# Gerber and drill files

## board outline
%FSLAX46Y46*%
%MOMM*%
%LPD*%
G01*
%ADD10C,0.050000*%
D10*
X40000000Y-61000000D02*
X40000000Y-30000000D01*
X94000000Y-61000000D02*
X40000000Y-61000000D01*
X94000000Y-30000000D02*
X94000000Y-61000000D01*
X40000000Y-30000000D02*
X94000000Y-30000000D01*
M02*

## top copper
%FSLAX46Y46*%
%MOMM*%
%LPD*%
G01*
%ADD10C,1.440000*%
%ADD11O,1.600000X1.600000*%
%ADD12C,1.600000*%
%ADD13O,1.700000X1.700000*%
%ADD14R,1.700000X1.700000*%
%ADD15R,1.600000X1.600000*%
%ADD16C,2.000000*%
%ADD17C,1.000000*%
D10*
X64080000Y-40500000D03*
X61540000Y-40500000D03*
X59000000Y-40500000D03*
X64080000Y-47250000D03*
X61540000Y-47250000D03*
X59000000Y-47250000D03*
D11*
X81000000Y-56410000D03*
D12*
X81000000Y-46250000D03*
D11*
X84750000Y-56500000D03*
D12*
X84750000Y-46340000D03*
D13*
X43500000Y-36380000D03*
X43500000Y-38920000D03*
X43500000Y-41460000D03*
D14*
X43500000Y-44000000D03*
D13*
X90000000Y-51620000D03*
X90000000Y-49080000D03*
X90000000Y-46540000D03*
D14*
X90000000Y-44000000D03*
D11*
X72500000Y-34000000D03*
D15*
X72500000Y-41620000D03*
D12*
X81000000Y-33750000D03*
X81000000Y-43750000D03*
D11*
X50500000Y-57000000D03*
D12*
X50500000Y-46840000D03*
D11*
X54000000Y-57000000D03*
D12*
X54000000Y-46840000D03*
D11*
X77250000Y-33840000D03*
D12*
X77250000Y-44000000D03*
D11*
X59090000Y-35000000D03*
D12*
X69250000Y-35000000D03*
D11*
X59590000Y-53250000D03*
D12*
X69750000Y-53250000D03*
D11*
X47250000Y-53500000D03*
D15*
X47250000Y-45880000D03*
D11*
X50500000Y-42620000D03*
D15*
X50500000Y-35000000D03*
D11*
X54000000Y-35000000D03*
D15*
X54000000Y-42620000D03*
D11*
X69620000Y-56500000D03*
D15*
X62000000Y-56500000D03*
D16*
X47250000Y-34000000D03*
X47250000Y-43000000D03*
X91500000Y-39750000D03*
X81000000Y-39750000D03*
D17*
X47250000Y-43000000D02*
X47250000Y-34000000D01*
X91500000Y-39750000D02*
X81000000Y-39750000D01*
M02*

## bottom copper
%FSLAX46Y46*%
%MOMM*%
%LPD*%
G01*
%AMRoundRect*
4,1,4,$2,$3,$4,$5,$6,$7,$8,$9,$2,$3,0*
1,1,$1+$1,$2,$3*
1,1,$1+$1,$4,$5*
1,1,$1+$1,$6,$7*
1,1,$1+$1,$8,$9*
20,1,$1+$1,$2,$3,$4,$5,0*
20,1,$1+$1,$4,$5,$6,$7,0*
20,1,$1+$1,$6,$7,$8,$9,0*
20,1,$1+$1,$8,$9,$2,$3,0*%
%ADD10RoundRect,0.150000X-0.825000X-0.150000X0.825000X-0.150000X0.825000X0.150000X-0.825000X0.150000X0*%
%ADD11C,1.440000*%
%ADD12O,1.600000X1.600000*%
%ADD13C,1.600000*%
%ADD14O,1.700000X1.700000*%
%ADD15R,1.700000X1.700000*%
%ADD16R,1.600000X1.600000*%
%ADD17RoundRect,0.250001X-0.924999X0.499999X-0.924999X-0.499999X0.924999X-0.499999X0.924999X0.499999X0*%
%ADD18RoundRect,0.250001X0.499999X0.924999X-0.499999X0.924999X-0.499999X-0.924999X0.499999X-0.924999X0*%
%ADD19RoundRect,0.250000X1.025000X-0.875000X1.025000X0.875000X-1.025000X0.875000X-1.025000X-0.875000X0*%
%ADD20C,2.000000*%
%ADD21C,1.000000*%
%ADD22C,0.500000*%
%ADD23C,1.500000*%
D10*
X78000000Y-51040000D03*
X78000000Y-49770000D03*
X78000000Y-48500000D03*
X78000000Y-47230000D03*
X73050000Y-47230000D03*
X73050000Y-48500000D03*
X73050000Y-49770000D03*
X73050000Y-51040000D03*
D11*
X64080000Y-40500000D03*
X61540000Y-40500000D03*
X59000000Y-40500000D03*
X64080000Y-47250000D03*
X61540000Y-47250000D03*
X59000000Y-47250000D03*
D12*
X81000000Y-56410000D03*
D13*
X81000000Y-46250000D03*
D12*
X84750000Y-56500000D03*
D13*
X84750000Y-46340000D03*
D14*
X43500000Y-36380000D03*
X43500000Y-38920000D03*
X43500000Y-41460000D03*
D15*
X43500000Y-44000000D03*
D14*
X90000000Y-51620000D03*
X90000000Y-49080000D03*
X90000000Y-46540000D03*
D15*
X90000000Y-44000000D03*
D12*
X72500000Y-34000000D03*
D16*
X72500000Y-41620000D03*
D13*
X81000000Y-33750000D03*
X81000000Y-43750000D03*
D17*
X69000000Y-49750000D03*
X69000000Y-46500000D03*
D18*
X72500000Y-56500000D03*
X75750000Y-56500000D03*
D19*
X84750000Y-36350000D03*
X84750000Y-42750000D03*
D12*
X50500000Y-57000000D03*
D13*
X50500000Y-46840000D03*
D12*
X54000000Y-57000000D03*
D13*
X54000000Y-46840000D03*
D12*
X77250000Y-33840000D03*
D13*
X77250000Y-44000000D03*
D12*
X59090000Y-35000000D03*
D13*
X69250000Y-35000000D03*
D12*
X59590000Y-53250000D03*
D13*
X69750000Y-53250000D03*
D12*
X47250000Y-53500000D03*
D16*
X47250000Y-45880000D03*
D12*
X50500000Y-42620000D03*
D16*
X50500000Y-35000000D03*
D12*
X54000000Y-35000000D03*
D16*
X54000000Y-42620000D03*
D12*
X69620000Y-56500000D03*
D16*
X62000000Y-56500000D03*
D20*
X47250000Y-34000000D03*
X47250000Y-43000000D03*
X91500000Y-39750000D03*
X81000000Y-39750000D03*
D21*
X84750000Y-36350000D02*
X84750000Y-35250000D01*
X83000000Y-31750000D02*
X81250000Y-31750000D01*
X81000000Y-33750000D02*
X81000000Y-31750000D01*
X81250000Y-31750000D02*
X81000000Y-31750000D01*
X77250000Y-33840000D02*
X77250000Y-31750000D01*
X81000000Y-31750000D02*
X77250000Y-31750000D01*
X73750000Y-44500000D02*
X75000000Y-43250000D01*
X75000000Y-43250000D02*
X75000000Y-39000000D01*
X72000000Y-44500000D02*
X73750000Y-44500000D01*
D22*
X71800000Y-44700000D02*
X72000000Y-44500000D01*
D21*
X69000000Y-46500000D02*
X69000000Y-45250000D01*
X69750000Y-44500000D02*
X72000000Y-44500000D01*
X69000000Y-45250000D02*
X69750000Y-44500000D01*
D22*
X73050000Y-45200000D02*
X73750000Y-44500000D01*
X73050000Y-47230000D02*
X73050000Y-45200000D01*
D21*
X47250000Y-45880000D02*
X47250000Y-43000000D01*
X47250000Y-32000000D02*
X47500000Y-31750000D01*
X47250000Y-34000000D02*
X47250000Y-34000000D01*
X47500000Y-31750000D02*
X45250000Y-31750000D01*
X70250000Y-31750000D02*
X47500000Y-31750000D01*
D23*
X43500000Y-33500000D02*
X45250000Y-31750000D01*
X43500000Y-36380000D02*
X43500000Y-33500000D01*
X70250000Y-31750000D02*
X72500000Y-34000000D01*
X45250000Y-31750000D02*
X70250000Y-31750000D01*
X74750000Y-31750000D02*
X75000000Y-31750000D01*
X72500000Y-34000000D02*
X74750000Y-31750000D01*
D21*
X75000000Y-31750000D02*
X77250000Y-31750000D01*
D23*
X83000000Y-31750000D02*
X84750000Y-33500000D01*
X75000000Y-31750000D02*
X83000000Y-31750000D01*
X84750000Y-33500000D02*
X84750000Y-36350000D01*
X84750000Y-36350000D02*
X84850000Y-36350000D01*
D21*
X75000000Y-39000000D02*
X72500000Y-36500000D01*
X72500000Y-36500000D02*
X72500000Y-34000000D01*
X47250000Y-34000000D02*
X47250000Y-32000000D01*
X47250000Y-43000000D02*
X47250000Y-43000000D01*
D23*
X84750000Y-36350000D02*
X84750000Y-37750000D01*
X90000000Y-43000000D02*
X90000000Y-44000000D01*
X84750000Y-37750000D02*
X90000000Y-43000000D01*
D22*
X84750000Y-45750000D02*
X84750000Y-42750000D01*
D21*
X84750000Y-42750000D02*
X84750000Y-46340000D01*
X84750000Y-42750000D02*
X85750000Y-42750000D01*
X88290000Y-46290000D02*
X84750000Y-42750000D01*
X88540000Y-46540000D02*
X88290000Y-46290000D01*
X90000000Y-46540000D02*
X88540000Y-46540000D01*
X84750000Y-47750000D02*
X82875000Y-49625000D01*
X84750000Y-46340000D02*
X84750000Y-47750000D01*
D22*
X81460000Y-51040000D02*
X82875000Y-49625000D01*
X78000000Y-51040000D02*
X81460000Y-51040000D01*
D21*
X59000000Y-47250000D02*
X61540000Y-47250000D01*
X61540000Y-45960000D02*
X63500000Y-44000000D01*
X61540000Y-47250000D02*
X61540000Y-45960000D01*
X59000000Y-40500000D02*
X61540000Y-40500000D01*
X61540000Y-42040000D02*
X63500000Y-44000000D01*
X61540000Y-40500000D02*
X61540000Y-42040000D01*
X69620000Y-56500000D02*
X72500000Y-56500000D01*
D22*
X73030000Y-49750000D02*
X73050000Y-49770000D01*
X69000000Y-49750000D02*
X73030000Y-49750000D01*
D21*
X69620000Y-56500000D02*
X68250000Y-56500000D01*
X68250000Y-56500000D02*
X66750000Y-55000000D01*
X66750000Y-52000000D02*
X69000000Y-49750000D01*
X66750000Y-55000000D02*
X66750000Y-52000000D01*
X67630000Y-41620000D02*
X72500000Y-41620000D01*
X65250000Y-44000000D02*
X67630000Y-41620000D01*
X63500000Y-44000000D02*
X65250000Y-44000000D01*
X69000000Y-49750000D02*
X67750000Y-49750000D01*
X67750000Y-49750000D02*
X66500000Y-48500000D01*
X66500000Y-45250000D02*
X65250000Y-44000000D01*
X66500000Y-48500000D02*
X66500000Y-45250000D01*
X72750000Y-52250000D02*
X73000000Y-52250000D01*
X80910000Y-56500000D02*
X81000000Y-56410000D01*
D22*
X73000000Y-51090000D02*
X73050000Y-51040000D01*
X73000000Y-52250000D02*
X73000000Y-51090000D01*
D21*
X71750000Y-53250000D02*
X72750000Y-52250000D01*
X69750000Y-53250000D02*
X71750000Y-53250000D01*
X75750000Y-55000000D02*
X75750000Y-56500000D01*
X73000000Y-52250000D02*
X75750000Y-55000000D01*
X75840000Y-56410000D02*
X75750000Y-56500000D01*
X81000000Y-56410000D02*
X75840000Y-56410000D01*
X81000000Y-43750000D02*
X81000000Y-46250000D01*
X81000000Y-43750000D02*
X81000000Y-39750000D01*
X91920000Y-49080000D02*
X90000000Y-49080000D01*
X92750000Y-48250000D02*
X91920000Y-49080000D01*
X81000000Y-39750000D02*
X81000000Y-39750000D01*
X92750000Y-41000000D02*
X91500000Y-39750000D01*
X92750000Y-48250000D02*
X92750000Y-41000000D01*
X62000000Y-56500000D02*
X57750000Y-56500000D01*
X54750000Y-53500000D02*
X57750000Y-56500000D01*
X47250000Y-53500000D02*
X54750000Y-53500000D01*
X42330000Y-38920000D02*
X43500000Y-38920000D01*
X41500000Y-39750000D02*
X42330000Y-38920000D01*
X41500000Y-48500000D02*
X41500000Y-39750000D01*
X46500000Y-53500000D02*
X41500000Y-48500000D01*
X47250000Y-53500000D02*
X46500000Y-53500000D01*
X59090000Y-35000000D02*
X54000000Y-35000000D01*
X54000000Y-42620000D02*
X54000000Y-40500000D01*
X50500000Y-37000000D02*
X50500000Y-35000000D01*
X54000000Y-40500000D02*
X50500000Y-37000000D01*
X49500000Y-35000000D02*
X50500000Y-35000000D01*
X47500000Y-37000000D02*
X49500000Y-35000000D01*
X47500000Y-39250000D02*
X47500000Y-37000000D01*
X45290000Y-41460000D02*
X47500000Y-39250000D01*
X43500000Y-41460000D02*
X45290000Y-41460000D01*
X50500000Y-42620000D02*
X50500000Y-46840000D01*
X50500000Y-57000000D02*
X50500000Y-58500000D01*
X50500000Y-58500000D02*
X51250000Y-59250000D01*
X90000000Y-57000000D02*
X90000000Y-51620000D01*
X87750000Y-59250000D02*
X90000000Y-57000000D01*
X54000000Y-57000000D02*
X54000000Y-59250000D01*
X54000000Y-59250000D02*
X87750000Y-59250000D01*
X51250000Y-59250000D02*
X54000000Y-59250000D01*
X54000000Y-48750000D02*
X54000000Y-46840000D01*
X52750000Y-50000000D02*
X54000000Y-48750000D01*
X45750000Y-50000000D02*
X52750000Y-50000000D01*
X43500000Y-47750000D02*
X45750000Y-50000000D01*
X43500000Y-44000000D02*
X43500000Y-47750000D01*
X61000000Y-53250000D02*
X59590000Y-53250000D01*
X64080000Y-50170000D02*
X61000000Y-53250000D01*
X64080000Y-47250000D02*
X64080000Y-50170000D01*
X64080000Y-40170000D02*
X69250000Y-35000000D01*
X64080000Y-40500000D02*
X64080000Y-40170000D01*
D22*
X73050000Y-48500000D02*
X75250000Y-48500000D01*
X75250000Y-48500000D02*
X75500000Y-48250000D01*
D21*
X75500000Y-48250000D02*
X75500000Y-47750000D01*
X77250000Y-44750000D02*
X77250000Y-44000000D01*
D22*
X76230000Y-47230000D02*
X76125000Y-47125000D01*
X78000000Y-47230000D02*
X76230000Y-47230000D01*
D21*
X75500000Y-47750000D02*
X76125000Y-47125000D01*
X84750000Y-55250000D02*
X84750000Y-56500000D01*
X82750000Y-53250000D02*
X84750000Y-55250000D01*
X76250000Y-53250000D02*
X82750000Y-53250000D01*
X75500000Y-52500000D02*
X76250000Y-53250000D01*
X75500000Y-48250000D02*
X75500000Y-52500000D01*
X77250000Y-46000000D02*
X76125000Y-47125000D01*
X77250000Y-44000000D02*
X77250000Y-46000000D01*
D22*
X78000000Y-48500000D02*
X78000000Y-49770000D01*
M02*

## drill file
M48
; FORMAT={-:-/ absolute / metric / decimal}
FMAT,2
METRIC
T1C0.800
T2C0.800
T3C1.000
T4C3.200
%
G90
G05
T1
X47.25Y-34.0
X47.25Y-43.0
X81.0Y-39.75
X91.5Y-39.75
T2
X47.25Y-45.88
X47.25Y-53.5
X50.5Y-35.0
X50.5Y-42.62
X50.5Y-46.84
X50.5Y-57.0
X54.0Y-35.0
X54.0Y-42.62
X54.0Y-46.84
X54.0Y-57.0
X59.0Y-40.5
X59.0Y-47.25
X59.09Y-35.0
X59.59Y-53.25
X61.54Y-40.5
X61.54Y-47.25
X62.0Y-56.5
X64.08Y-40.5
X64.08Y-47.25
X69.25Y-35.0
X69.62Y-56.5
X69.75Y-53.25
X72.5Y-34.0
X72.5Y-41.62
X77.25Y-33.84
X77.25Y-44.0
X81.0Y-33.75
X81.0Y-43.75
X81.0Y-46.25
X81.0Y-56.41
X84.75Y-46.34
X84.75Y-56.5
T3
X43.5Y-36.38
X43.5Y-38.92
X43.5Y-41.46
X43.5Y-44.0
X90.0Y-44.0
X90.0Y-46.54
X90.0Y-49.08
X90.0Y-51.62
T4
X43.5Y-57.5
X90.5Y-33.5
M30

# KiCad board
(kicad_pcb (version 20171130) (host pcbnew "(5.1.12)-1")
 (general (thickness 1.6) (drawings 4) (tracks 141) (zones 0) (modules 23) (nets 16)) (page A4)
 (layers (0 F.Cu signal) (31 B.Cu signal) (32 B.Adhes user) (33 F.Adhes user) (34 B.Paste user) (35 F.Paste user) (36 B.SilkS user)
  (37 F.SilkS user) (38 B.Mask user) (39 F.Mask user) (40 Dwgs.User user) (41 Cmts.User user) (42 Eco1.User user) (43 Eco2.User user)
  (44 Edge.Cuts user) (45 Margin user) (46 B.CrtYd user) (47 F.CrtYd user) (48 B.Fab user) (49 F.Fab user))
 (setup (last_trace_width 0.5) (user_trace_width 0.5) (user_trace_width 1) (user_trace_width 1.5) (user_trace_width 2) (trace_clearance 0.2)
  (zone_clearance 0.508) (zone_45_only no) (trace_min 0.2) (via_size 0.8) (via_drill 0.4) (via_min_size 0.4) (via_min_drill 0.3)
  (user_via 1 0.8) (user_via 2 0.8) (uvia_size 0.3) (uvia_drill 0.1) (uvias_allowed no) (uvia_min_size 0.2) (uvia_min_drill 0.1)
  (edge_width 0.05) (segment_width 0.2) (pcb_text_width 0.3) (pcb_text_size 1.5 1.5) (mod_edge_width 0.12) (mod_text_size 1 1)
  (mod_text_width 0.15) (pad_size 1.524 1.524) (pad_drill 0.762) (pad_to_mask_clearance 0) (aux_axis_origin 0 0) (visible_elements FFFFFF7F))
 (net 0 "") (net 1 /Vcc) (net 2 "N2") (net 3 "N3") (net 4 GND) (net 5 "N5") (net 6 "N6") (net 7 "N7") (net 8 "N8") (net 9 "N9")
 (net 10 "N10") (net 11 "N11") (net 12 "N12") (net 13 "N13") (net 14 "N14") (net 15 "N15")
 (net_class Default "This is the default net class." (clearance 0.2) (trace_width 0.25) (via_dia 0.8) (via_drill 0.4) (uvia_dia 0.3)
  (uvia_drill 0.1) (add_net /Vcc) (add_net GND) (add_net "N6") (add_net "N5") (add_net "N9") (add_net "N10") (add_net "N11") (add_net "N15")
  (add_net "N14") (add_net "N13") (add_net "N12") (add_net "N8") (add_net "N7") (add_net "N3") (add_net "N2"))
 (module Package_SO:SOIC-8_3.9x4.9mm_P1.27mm (layer B.Cu) (at 75.525 49.135)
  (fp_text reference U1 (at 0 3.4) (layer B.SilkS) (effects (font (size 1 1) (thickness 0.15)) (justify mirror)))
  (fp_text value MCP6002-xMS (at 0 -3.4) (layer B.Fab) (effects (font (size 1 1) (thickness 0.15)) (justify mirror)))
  (pad 8 smd roundrect (at 2.475 1.905) (size 1.95 0.6) (layers B.Cu B.Paste B.Mask) (roundrect_rratio 0.25) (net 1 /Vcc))
  (pad 7 smd roundrect (at 2.475 0.635) (size 1.95 0.6) (layers B.Cu B.Paste B.Mask) (roundrect_rratio 0.25) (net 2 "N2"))
  (pad 6 smd roundrect (at 2.475 -0.635) (size 1.95 0.6) (layers B.Cu B.Paste B.Mask) (roundrect_rratio 0.25) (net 2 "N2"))
  (pad 5 smd roundrect (at 2.475 -1.905) (size 1.95 0.6) (layers B.Cu B.Paste B.Mask) (roundrect_rratio 0.25) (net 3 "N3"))
  (pad 4 smd roundrect (at -2.475 -1.905) (size 1.95 0.6) (layers B.Cu B.Paste B.Mask) (roundrect_rratio 0.25) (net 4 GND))
  (pad 3 smd roundrect (at -2.475 -0.635) (size 1.95 0.6) (layers B.Cu B.Paste B.Mask) (roundrect_rratio 0.25) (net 3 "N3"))
  (pad 2 smd roundrect (at -2.475 0.635) (size 1.95 0.6) (layers B.Cu B.Paste B.Mask) (roundrect_rratio 0.25) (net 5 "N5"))
  (pad 1 smd roundrect (at -2.475 1.905) (size 1.95 0.6) (layers B.Cu B.Paste B.Mask) (roundrect_rratio 0.25) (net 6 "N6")))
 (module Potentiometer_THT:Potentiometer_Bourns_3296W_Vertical (layer F.Cu) (at 59 40.5 180)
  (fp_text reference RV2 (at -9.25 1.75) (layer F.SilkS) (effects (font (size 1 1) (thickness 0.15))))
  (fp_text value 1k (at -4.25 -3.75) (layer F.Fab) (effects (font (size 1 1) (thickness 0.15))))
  (pad 3 thru_hole circle (at -5.08 0 180) (size 1.44 1.44) (drill 0.8) (layers *.Cu *.Mask) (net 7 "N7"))
  (pad 2 thru_hole circle (at -2.54 0 180) (size 1.44 1.44) (drill 0.8) (layers *.Cu *.Mask) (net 5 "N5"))
  (pad 1 thru_hole circle (at 0 0 180) (size 1.44 1.44) (drill 0.8) (layers *.Cu *.Mask) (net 5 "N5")))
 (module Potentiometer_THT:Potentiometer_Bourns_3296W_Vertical (layer F.Cu) (at 59 47.25 180)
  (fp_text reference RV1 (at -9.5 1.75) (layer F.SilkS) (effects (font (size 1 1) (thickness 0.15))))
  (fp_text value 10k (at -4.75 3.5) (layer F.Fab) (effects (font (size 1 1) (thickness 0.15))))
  (pad 3 thru_hole circle (at -5.08 0 180) (size 1.44 1.44) (drill 0.8) (layers *.Cu *.Mask) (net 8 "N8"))
  (pad 2 thru_hole circle (at -2.54 0 180) (size 1.44 1.44) (drill 0.8) (layers *.Cu *.Mask) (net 5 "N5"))
  (pad 1 thru_hole circle (at 0 0 180) (size 1.44 1.44) (drill 0.8) (layers *.Cu *.Mask) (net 5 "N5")))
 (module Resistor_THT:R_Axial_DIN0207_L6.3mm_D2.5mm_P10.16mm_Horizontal (layer F.Cu) (at 81 46.25 270)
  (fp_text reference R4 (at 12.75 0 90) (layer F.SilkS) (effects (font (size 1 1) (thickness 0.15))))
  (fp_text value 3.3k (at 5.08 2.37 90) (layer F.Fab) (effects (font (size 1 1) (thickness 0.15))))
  (pad 2 thru_hole oval (at 10.16 0 270) (size 1.6 1.6) (drill 0.8) (layers *.Cu *.Mask) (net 6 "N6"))
  (pad 1 thru_hole circle (at 0 0 270) (size 1.6 1.6) (drill 0.8) (layers *.Cu *.Mask) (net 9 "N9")))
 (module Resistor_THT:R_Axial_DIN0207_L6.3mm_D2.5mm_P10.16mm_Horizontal (layer F.Cu) (at 84.75 46.34 270)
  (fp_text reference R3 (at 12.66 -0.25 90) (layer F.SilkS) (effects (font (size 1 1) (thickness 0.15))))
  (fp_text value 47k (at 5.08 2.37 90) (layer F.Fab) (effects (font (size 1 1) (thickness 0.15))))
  (pad 2 thru_hole oval (at 10.16 0 270) (size 1.6 1.6) (drill 0.8) (layers *.Cu *.Mask) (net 3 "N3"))
  (pad 1 thru_hole circle (at 0 0 270) (size 1.6 1.6) (drill 0.8) (layers *.Cu *.Mask) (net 1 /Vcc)))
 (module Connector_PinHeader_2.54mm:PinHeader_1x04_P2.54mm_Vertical (layer F.Cu) (at 43.5 44 180)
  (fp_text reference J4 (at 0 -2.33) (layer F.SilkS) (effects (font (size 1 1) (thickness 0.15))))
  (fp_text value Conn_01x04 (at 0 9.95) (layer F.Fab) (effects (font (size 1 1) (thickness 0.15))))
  (pad 4 thru_hole oval (at 0 7.62 180) (size 1.7 1.7) (drill 1) (layers *.Cu *.Mask) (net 4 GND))
  (pad 3 thru_hole oval (at 0 5.08 180) (size 1.7 1.7) (drill 1) (layers *.Cu *.Mask) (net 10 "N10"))
  (pad 2 thru_hole oval (at 0 2.54 180) (size 1.7 1.7) (drill 1) (layers *.Cu *.Mask) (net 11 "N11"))
  (pad 1 thru_hole rect (at 0 0 180) (size 1.7 1.7) (drill 1) (layers *.Cu *.Mask) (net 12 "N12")))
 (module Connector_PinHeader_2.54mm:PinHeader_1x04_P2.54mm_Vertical (layer F.Cu) (at 90 44)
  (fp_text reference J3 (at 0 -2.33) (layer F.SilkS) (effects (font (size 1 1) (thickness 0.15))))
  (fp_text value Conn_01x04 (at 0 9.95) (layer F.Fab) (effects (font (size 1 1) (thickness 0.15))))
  (pad 4 thru_hole oval (at 0 7.62) (size 1.7 1.7) (drill 1) (layers *.Cu *.Mask) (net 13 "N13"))
  (pad 3 thru_hole oval (at 0 5.08) (size 1.7 1.7) (drill 1) (layers *.Cu *.Mask) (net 9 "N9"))
  (pad 2 thru_hole oval (at 0 2.54) (size 1.7 1.7) (drill 1) (layers *.Cu *.Mask) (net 1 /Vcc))
  (pad 1 thru_hole rect (at 0 0) (size 1.7 1.7) (drill 1) (layers *.Cu *.Mask) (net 4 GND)))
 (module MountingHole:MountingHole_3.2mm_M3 (layer F.Cu) (at 90.5 33.5)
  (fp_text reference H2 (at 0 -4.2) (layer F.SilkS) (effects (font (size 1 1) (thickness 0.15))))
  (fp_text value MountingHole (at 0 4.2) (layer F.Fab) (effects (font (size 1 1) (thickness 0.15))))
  (pad 1 np_thru_hole circle (at 0 0) (size 3.2 3.2) (drill 3.2) (layers *.Cu *.Mask)))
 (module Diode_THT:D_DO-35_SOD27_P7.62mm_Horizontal (layer F.Cu) (at 72.5 41.62 90)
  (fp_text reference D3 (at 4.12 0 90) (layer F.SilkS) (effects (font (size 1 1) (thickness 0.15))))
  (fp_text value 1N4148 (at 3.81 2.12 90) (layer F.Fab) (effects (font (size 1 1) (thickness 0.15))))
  (pad 2 thru_hole oval (at 7.62 0 90) (size 1.6 1.6) (drill 0.8) (layers *.Cu *.Mask) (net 4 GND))
  (pad 1 thru_hole rect (at 0 0 90) (size 1.6 1.6) (drill 0.8) (layers *.Cu *.Mask) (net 5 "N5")))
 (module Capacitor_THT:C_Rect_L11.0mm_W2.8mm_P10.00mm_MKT (layer F.Cu) (at 81 43.75 90)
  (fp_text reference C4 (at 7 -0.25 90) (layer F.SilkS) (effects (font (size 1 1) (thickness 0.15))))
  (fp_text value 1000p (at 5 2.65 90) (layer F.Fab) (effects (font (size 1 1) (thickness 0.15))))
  (pad 2 thru_hole circle (at 10 0 90) (size 1.6 1.6) (drill 0.8) (layers *.Cu *.Mask) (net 4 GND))
  (pad 1 thru_hole circle (at 0 0 90) (size 1.6 1.6) (drill 0.8) (layers *.Cu *.Mask) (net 9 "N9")))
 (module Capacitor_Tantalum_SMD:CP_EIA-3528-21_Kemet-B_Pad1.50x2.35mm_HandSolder (layer B.Cu) (at 69 48.125 270)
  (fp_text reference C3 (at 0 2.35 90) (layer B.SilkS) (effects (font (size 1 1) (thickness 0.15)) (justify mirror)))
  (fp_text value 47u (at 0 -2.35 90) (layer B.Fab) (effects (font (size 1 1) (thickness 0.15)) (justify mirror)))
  (pad 2 smd roundrect (at 1.625 0 270) (size 1.5 2.35) (layers B.Cu B.Paste B.Mask) (roundrect_rratio 0.166667) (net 5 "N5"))
  (pad 1 smd roundrect (at -1.625 0 270) (size 1.5 2.35) (layers B.Cu B.Paste B.Mask) (roundrect_rratio 0.166667) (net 4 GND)))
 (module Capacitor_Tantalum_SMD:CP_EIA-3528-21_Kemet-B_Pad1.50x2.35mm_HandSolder (layer B.Cu) (at 74.125 56.5 180)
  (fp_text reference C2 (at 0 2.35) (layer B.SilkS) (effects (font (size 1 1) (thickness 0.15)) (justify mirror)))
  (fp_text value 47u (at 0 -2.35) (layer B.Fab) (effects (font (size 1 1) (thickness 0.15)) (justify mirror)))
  (pad 2 smd roundrect (at 1.625 0 180) (size 1.5 2.35) (layers B.Cu B.Paste B.Mask) (roundrect_rratio 0.166667) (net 5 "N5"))
  (pad 1 smd roundrect (at -1.625 0 180) (size 1.5 2.35) (layers B.Cu B.Paste B.Mask) (roundrect_rratio 0.166667) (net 6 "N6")))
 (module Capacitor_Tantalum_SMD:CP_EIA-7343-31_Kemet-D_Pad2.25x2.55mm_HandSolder (layer B.Cu) (at 84.75 39.55 90)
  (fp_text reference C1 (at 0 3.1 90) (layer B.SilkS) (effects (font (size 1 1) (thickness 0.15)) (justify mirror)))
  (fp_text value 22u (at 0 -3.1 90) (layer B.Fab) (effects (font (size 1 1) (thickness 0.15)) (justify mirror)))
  (pad 2 smd roundrect (at 3.2 0 90) (size 2.25 2.55) (layers B.Cu B.Paste B.Mask) (roundrect_rratio 0.111111) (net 4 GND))
  (pad 1 smd roundrect (at -3.2 0 90) (size 2.25 2.55) (layers B.Cu B.Paste B.Mask) (roundrect_rratio 0.111111) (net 1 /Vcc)))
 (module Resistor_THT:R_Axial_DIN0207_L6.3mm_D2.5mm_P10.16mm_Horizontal (layer F.Cu) (at 50.5 46.84 270)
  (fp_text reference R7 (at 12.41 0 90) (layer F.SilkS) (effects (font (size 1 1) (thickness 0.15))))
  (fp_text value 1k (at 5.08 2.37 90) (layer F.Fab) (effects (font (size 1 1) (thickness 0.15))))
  (pad 2 thru_hole oval (at 10.16 0 270) (size 1.6 1.6) (drill 0.8) (layers *.Cu *.Mask) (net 13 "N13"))
  (pad 1 thru_hole circle (at 0 0 270) (size 1.6 1.6) (drill 0.8) (layers *.Cu *.Mask) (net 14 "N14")))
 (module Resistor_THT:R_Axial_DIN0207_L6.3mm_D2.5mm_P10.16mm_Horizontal (layer F.Cu) (at 54 46.84 270)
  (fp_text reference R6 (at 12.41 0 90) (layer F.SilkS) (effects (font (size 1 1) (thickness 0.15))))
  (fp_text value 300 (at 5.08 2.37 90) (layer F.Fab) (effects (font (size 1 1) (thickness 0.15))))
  (pad 2 thru_hole oval (at 10.16 0 270) (size 1.6 1.6) (drill 0.8) (layers *.Cu *.Mask) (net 13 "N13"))
  (pad 1 thru_hole circle (at 0 0 270) (size 1.6 1.6) (drill 0.8) (layers *.Cu *.Mask) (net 12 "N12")))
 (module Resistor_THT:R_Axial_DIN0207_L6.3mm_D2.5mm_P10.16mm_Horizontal (layer F.Cu) (at 77.25 44 90)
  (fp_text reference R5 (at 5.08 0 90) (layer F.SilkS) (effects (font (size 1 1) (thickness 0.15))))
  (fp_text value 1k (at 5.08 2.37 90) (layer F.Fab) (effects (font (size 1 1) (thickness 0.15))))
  (pad 2 thru_hole oval (at 10.16 0 90) (size 1.6 1.6) (drill 0.8) (layers *.Cu *.Mask) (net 4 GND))
  (pad 1 thru_hole circle (at 0 0 90) (size 1.6 1.6) (drill 0.8) (layers *.Cu *.Mask) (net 3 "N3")))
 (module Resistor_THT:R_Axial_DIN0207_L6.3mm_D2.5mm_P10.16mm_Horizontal (layer F.Cu) (at 69.25 35 180)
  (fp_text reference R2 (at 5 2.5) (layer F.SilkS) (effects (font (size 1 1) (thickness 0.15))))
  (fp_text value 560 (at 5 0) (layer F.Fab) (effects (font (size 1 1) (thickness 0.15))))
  (pad 2 thru_hole oval (at 10.16 0 180) (size 1.6 1.6) (drill 0.8) (layers *.Cu *.Mask) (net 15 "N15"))
  (pad 1 thru_hole circle (at 0 0 180) (size 1.6 1.6) (drill 0.8) (layers *.Cu *.Mask) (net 7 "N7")))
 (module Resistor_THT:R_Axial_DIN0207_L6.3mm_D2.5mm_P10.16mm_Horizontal (layer F.Cu) (at 69.75 53.25 180)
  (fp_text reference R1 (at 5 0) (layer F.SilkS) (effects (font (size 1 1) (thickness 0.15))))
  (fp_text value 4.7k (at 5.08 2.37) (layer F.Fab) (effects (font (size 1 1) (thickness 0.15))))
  (pad 2 thru_hole oval (at 10.16 0 180) (size 1.6 1.6) (drill 0.8) (layers *.Cu *.Mask) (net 8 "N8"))
  (pad 1 thru_hole circle (at 0 0 180) (size 1.6 1.6) (drill 0.8) (layers *.Cu *.Mask) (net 6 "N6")))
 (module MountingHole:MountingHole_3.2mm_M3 (layer F.Cu) (at 43.5 57.5)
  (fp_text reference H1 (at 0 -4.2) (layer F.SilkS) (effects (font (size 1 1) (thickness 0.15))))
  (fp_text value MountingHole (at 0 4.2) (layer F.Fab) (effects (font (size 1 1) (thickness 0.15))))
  (pad 1 np_thru_hole circle (at 0 0) (size 3.2 3.2) (drill 3.2) (layers *.Cu *.Mask)))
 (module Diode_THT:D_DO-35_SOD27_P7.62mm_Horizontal (layer F.Cu) (at 47.25 45.88 270)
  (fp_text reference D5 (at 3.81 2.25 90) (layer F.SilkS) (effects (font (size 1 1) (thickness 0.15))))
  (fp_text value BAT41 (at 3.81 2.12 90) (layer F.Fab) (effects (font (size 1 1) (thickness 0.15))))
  (pad 2 thru_hole oval (at 7.62 0 270) (size 1.6 1.6) (drill 0.8) (layers *.Cu *.Mask) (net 10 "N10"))
  (pad 1 thru_hole rect (at 0 0 270) (size 1.6 1.6) (drill 0.8) (layers *.Cu *.Mask) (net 4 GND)))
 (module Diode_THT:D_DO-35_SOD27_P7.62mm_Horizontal (layer F.Cu) (at 50.5 35 270)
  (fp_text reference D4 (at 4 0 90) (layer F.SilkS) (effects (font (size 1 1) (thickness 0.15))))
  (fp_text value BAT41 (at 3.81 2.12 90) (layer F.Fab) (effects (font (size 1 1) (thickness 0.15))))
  (pad 2 thru_hole oval (at 7.62 0 270) (size 1.6 1.6) (drill 0.8) (layers *.Cu *.Mask) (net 14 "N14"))
  (pad 1 thru_hole rect (at 0 0 270) (size 1.6 1.6) (drill 0.8) (layers *.Cu *.Mask) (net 11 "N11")))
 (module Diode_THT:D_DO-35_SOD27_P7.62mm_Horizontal (layer F.Cu) (at 54 42.62 90)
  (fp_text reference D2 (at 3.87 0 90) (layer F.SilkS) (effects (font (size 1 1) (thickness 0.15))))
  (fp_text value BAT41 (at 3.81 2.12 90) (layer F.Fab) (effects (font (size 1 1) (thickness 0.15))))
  (pad 2 thru_hole oval (at 7.62 0 90) (size 1.6 1.6) (drill 0.8) (layers *.Cu *.Mask) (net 15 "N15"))
  (pad 1 thru_hole rect (at 0 0 90) (size 1.6 1.6) (drill 0.8) (layers *.Cu *.Mask) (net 11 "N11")))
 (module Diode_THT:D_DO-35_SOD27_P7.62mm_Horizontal (layer F.Cu) (at 62 56.5)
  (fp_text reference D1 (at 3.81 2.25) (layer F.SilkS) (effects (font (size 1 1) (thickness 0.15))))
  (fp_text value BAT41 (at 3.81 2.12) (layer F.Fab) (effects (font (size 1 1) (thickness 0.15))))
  (pad 2 thru_hole oval (at 7.62 0) (size 1.6 1.6) (drill 0.8) (layers *.Cu *.Mask) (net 5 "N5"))
  (pad 1 thru_hole rect (at 0 0) (size 1.6 1.6) (drill 0.8) (layers *.Cu *.Mask) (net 10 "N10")))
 (gr_line (start 40 61) (end 40 30) (layer Edge.Cuts) (width 0.05))
 (gr_line (start 94 61) (end 40 61) (layer Edge.Cuts) (width 0.05))
 (gr_line (start 94 30) (end 94 61) (layer Edge.Cuts) (width 0.05))
 (gr_line (start 40 30) (end 94 30) (layer Edge.Cuts) (width 0.05))
 (segment (start 84.75 36.35) (end 84.75 35.25) (width 1) (layer B.Cu) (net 4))
 (segment (start 83 31.75) (end 81.25 31.75) (width 1) (layer B.Cu) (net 4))
 (segment (start 81 33.75) (end 81 31.75) (width 1) (layer B.Cu) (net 4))
 (segment (start 81.25 31.75) (end 81 31.75) (width 1) (layer B.Cu) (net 4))
 (segment (start 77.25 33.84) (end 77.25 31.75) (width 1) (layer B.Cu) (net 4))
 (segment (start 81 31.75) (end 77.25 31.75) (width 1) (layer B.Cu) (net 4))
 (segment (start 73.75 44.5) (end 75 43.25) (width 1) (layer B.Cu) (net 4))
 (segment (start 75 43.25) (end 75 39) (width 1) (layer B.Cu) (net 4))
 (segment (start 72 44.5) (end 73.75 44.5) (width 1) (layer B.Cu) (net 4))
 (segment (start 71.8 44.7) (end 72 44.5) (width 0.5) (layer B.Cu) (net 4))
 (segment (start 69 46.5) (end 69 45.25) (width 1) (layer B.Cu) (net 4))
 (segment (start 69.75 44.5) (end 72 44.5) (width 1) (layer B.Cu) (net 4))
 (segment (start 69 45.25) (end 69.75 44.5) (width 1) (layer B.Cu) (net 4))
 (segment (start 73.05 45.2) (end 73.75 44.5) (width 0.5) (layer B.Cu) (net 4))
 (segment (start 73.05 47.23) (end 73.05 45.2) (width 0.5) (layer B.Cu) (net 4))
 (segment (start 47.25 45.88) (end 47.25 43) (width 1) (layer B.Cu) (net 4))
 (segment (start 47.25 43) (end 47.25 34) (width 1) (layer F.Cu) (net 4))
 (segment (start 47.25 32) (end 47.5 31.75) (width 1) (layer B.Cu) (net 4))
 (segment (start 47.25 34) (end 47.25 34) (width 1) (layer B.Cu) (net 4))
 (segment (start 47.5 31.75) (end 45.25 31.75) (width 1) (layer B.Cu) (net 4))
 (segment (start 70.25 31.75) (end 47.5 31.75) (width 1) (layer B.Cu) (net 4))
 (segment (start 43.5 33.5) (end 45.25 31.75) (width 1.5) (layer B.Cu) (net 4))
 (segment (start 43.5 36.38) (end 43.5 33.5) (width 1.5) (layer B.Cu) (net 4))
 (segment (start 70.25 31.75) (end 72.5 34) (width 1.5) (layer B.Cu) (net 4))
 (segment (start 45.25 31.75) (end 70.25 31.75) (width 1.5) (layer B.Cu) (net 4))
 (segment (start 74.75 31.75) (end 75 31.75) (width 1.5) (layer B.Cu) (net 4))
 (segment (start 72.5 34) (end 74.75 31.75) (width 1.5) (layer B.Cu) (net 4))
 (segment (start 75 31.75) (end 77.25 31.75) (width 1) (layer B.Cu) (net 4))
 (segment (start 83 31.75) (end 84.75 33.5) (width 1.5) (layer B.Cu) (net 4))
 (segment (start 75 31.75) (end 83 31.75) (width 1.5) (layer B.Cu) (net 4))
 (segment (start 84.75 33.5) (end 84.75 36.35) (width 1.5) (layer B.Cu) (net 4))
 (segment (start 84.75 36.35) (end 84.85 36.35) (width 1.5) (layer B.Cu) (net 4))
 (segment (start 75 39) (end 72.5 36.5) (width 1) (layer B.Cu) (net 4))
 (segment (start 72.5 36.5) (end 72.5 34) (width 1) (layer B.Cu) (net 4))
 (segment (start 47.25 34) (end 47.25 32) (width 1) (layer B.Cu) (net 4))
 (via (at 47.25 34) (size 2) (drill 0.8) (layers F.Cu B.Cu) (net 4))
 (segment (start 47.25 43) (end 47.25 43) (width 1) (layer B.Cu) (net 4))
 (via (at 47.25 43) (size 2) (drill 0.8) (layers F.Cu B.Cu) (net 4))
 (segment (start 84.75 36.35) (end 84.75 37.75) (width 1.5) (layer B.Cu) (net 4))
 (segment (start 90 43) (end 90 44) (width 1.5) (layer B.Cu) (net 4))
 (segment (start 84.75 37.75) (end 90 43) (width 1.5) (layer B.Cu) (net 4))
 (segment (start 84.75 45.75) (end 84.75 42.75) (width 0.5) (layer B.Cu) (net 1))
 (segment (start 84.75 42.75) (end 84.75 46.34) (width 1) (layer B.Cu) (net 1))
 (segment (start 84.75 42.75) (end 85.75 42.75) (width 1) (layer B.Cu) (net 1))
 (segment (start 88.29 46.29) (end 84.75 42.75) (width 1) (layer B.Cu) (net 1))
 (segment (start 88.54 46.54) (end 88.29 46.29) (width 1) (layer B.Cu) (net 1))
 (segment (start 90 46.54) (end 88.54 46.54) (width 1) (layer B.Cu) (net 1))
 (segment (start 84.75 47.75) (end 82.875 49.625) (width 1) (layer B.Cu) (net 1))
 (segment (start 84.75 46.34) (end 84.75 47.75) (width 1) (layer B.Cu) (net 1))
 (segment (start 81.46 51.04) (end 82.875 49.625) (width 0.5) (layer B.Cu) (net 1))
 (segment (start 78 51.04) (end 81.46 51.04) (width 0.5) (layer B.Cu) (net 1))
 (segment (start 59 47.25) (end 61.54 47.25) (width 1) (layer B.Cu) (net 5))
 (segment (start 61.54 45.96) (end 63.5 44) (width 1) (layer B.Cu) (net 5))
 (segment (start 61.54 47.25) (end 61.54 45.96) (width 1) (layer B.Cu) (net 5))
 (segment (start 59 40.5) (end 61.54 40.5) (width 1) (layer B.Cu) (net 5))
 (segment (start 61.54 42.04) (end 63.5 44) (width 1) (layer B.Cu) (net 5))
 (segment (start 61.54 40.5) (end 61.54 42.04) (width 1) (layer B.Cu) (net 5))
 (segment (start 69.62 56.5) (end 72.5 56.5) (width 1) (layer B.Cu) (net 5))
 (segment (start 73.03 49.75) (end 73.05 49.77) (width 0.5) (layer B.Cu) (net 5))
 (segment (start 69 49.75) (end 73.03 49.75) (width 0.5) (layer B.Cu) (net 5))
 (segment (start 69.62 56.5) (end 68.25 56.5) (width 1) (layer B.Cu) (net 5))
 (segment (start 68.25 56.5) (end 66.75 55) (width 1) (layer B.Cu) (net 5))
 (segment (start 66.75 52) (end 69 49.75) (width 1) (layer B.Cu) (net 5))
 (segment (start 66.75 55) (end 66.75 52) (width 1) (layer B.Cu) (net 5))
 (segment (start 67.63 41.62) (end 72.5 41.62) (width 1) (layer B.Cu) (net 5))
 (segment (start 65.25 44) (end 67.63 41.62) (width 1) (layer B.Cu) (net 5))
 (segment (start 63.5 44) (end 65.25 44) (width 1) (layer B.Cu) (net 5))
 (segment (start 69 49.75) (end 67.75 49.75) (width 1) (layer B.Cu) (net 5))
 (segment (start 67.75 49.75) (end 66.5 48.5) (width 1) (layer B.Cu) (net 5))
 (segment (start 66.5 45.25) (end 65.25 44) (width 1) (layer B.Cu) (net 5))
 (segment (start 66.5 48.5) (end 66.5 45.25) (width 1) (layer B.Cu) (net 5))
 (segment (start 72.75 52.25) (end 73 52.25) (width 1) (layer B.Cu) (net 6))
 (segment (start 80.91 56.5) (end 81 56.41) (width 1) (layer B.Cu) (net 6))
 (segment (start 73 51.09) (end 73.05 51.04) (width 0.5) (layer B.Cu) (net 6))
 (segment (start 73 52.25) (end 73 51.09) (width 0.5) (layer B.Cu) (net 6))
 (segment (start 71.75 53.25) (end 72.75 52.25) (width 1) (layer B.Cu) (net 6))
 (segment (start 69.75 53.25) (end 71.75 53.25) (width 1) (layer B.Cu) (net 6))
 (segment (start 75.75 55) (end 75.75 56.5) (width 1) (layer B.Cu) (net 6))
 (segment (start 73 52.25) (end 75.75 55) (width 1) (layer B.Cu) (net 6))
 (segment (start 75.84 56.41) (end 75.75 56.5) (width 1) (layer B.Cu) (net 6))
 (segment (start 81 56.41) (end 75.84 56.41) (width 1) (layer B.Cu) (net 6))
 (segment (start 81 43.75) (end 81 46.25) (width 1) (layer B.Cu) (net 9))
 (segment (start 81 43.75) (end 81 39.75) (width 1) (layer B.Cu) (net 9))
 (segment (start 91.92 49.08) (end 90 49.08) (width 1) (layer B.Cu) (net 9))
 (segment (start 92.75 48.25) (end 91.92 49.08) (width 1) (layer B.Cu) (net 9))
 (via (at 91.5 39.75) (size 2) (drill 0.8) (layers F.Cu B.Cu) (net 9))
 (segment (start 81 39.75) (end 81 39.75) (width 1) (layer B.Cu) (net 9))
 (via (at 81 39.75) (size 2) (drill 0.8) (layers F.Cu B.Cu) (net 9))
 (segment (start 92.75 41) (end 91.5 39.75) (width 1) (layer B.Cu) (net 9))
 (segment (start 92.75 48.25) (end 92.75 41) (width 1) (layer B.Cu) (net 9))
 (segment (start 91.5 39.75) (end 81 39.75) (width 1) (layer F.Cu) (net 9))
 (segment (start 62 56.5) (end 57.75 56.5) (width 1) (layer B.Cu) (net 10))
 (segment (start 54.75 53.5) (end 57.75 56.5) (width 1) (layer B.Cu) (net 10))
 (segment (start 47.25 53.5) (end 54.75 53.5) (width 1) (layer B.Cu) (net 10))
 (segment (start 42.33 38.92) (end 43.5 38.92) (width 1) (layer B.Cu) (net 10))
 (segment (start 41.5 39.75) (end 42.33 38.92) (width 1) (layer B.Cu) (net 10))
 (segment (start 41.5 48.5) (end 41.5 39.75) (width 1) (layer B.Cu) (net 10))
 (segment (start 46.5 53.5) (end 41.5 48.5) (width 1) (layer B.Cu) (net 10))
 (segment (start 47.25 53.5) (end 46.5 53.5) (width 1) (layer B.Cu) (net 10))
 (segment (start 59.09 35) (end 54 35) (width 1) (layer B.Cu) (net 15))
 (segment (start 54 42.62) (end 54 40.5) (width 1) (layer B.Cu) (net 11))
 (segment (start 50.5 37) (end 50.5 35) (width 1) (layer B.Cu) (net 11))
 (segment (start 54 40.5) (end 50.5 37) (width 1) (layer B.Cu) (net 11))
 (segment (start 49.5 35) (end 50.5 35) (width 1) (layer B.Cu) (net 11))
 (segment (start 47.5 37) (end 49.5 35) (width 1) (layer B.Cu) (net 11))
 (segment (start 47.5 39.25) (end 47.5 37) (width 1) (layer B.Cu) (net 11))
 (segment (start 45.29 41.46) (end 47.5 39.25) (width 1) (layer B.Cu) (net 11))
 (segment (start 43.5 41.46) (end 45.29 41.46) (width 1) (layer B.Cu) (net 11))
 (segment (start 50.5 42.62) (end 50.5 46.84) (width 1) (layer B.Cu) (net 14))
 (segment (start 50.5 57) (end 50.5 58.5) (width 1) (layer B.Cu) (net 13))
 (segment (start 50.5 58.5) (end 51.25 59.25) (width 1) (layer B.Cu) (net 13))
 (segment (start 90 57) (end 90 51.62) (width 1) (layer B.Cu) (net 13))
 (segment (start 87.75 59.25) (end 90 57) (width 1) (layer B.Cu) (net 13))
 (segment (start 54 57) (end 54 59.25) (width 1) (layer B.Cu) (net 13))
 (segment (start 54 59.25) (end 87.75 59.25) (width 1) (layer B.Cu) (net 13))
 (segment (start 51.25 59.25) (end 54 59.25) (width 1) (layer B.Cu) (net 13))
 (segment (start 54 48.75) (end 54 46.84) (width 1) (layer B.Cu) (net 12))
 (segment (start 52.75 50) (end 54 48.75) (width 1) (layer B.Cu) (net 12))
 (segment (start 45.75 50) (end 52.75 50) (width 1) (layer B.Cu) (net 12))
 (segment (start 43.5 47.75) (end 45.75 50) (width 1) (layer B.Cu) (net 12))
 (segment (start 43.5 44) (end 43.5 47.75) (width 1) (layer B.Cu) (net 12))
 (segment (start 61 53.25) (end 59.59 53.25) (width 1) (layer B.Cu) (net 8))
 (segment (start 64.08 50.17) (end 61 53.25) (width 1) (layer B.Cu) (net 8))
 (segment (start 64.08 47.25) (end 64.08 50.17) (width 1) (layer B.Cu) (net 8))
 (segment (start 64.08 40.17) (end 69.25 35) (width 1) (layer B.Cu) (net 7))
 (segment (start 64.08 40.5) (end 64.08 40.17) (width 1) (layer B.Cu) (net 7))
 (segment (start 73.05 48.5) (end 75.25 48.5) (width 0.5) (layer B.Cu) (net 3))
 (segment (start 75.25 48.5) (end 75.5 48.25) (width 0.5) (layer B.Cu) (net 3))
 (segment (start 75.5 48.25) (end 75.5 47.75) (width 1) (layer B.Cu) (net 3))
 (segment (start 77.25 44.75) (end 77.25 44) (width 1) (layer B.Cu) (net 3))
 (segment (start 76.23 47.23) (end 76.125 47.125) (width 0.5) (layer B.Cu) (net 3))
 (segment (start 78 47.23) (end 76.23 47.23) (width 0.5) (layer B.Cu) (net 3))
 (segment (start 75.5 47.75) (end 76.125 47.125) (width 1) (layer B.Cu) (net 3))
 (segment (start 84.75 55.25) (end 84.75 56.5) (width 1) (layer B.Cu) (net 3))
 (segment (start 82.75 53.25) (end 84.75 55.25) (width 1) (layer B.Cu) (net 3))
 (segment (start 76.25 53.25) (end 82.75 53.25) (width 1) (layer B.Cu) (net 3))
 (segment (start 75.5 52.5) (end 76.25 53.25) (width 1) (layer B.Cu) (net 3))
 (segment (start 75.5 48.25) (end 75.5 52.5) (width 1) (layer B.Cu) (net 3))
 (segment (start 77.25 46) (end 76.125 47.125) (width 1) (layer B.Cu) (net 3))
 (segment (start 77.25 44) (end 77.25 46) (width 1) (layer B.Cu) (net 3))
 (segment (start 78 48.5) (end 78 49.77) (width 0.5) (layer B.Cu) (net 2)))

